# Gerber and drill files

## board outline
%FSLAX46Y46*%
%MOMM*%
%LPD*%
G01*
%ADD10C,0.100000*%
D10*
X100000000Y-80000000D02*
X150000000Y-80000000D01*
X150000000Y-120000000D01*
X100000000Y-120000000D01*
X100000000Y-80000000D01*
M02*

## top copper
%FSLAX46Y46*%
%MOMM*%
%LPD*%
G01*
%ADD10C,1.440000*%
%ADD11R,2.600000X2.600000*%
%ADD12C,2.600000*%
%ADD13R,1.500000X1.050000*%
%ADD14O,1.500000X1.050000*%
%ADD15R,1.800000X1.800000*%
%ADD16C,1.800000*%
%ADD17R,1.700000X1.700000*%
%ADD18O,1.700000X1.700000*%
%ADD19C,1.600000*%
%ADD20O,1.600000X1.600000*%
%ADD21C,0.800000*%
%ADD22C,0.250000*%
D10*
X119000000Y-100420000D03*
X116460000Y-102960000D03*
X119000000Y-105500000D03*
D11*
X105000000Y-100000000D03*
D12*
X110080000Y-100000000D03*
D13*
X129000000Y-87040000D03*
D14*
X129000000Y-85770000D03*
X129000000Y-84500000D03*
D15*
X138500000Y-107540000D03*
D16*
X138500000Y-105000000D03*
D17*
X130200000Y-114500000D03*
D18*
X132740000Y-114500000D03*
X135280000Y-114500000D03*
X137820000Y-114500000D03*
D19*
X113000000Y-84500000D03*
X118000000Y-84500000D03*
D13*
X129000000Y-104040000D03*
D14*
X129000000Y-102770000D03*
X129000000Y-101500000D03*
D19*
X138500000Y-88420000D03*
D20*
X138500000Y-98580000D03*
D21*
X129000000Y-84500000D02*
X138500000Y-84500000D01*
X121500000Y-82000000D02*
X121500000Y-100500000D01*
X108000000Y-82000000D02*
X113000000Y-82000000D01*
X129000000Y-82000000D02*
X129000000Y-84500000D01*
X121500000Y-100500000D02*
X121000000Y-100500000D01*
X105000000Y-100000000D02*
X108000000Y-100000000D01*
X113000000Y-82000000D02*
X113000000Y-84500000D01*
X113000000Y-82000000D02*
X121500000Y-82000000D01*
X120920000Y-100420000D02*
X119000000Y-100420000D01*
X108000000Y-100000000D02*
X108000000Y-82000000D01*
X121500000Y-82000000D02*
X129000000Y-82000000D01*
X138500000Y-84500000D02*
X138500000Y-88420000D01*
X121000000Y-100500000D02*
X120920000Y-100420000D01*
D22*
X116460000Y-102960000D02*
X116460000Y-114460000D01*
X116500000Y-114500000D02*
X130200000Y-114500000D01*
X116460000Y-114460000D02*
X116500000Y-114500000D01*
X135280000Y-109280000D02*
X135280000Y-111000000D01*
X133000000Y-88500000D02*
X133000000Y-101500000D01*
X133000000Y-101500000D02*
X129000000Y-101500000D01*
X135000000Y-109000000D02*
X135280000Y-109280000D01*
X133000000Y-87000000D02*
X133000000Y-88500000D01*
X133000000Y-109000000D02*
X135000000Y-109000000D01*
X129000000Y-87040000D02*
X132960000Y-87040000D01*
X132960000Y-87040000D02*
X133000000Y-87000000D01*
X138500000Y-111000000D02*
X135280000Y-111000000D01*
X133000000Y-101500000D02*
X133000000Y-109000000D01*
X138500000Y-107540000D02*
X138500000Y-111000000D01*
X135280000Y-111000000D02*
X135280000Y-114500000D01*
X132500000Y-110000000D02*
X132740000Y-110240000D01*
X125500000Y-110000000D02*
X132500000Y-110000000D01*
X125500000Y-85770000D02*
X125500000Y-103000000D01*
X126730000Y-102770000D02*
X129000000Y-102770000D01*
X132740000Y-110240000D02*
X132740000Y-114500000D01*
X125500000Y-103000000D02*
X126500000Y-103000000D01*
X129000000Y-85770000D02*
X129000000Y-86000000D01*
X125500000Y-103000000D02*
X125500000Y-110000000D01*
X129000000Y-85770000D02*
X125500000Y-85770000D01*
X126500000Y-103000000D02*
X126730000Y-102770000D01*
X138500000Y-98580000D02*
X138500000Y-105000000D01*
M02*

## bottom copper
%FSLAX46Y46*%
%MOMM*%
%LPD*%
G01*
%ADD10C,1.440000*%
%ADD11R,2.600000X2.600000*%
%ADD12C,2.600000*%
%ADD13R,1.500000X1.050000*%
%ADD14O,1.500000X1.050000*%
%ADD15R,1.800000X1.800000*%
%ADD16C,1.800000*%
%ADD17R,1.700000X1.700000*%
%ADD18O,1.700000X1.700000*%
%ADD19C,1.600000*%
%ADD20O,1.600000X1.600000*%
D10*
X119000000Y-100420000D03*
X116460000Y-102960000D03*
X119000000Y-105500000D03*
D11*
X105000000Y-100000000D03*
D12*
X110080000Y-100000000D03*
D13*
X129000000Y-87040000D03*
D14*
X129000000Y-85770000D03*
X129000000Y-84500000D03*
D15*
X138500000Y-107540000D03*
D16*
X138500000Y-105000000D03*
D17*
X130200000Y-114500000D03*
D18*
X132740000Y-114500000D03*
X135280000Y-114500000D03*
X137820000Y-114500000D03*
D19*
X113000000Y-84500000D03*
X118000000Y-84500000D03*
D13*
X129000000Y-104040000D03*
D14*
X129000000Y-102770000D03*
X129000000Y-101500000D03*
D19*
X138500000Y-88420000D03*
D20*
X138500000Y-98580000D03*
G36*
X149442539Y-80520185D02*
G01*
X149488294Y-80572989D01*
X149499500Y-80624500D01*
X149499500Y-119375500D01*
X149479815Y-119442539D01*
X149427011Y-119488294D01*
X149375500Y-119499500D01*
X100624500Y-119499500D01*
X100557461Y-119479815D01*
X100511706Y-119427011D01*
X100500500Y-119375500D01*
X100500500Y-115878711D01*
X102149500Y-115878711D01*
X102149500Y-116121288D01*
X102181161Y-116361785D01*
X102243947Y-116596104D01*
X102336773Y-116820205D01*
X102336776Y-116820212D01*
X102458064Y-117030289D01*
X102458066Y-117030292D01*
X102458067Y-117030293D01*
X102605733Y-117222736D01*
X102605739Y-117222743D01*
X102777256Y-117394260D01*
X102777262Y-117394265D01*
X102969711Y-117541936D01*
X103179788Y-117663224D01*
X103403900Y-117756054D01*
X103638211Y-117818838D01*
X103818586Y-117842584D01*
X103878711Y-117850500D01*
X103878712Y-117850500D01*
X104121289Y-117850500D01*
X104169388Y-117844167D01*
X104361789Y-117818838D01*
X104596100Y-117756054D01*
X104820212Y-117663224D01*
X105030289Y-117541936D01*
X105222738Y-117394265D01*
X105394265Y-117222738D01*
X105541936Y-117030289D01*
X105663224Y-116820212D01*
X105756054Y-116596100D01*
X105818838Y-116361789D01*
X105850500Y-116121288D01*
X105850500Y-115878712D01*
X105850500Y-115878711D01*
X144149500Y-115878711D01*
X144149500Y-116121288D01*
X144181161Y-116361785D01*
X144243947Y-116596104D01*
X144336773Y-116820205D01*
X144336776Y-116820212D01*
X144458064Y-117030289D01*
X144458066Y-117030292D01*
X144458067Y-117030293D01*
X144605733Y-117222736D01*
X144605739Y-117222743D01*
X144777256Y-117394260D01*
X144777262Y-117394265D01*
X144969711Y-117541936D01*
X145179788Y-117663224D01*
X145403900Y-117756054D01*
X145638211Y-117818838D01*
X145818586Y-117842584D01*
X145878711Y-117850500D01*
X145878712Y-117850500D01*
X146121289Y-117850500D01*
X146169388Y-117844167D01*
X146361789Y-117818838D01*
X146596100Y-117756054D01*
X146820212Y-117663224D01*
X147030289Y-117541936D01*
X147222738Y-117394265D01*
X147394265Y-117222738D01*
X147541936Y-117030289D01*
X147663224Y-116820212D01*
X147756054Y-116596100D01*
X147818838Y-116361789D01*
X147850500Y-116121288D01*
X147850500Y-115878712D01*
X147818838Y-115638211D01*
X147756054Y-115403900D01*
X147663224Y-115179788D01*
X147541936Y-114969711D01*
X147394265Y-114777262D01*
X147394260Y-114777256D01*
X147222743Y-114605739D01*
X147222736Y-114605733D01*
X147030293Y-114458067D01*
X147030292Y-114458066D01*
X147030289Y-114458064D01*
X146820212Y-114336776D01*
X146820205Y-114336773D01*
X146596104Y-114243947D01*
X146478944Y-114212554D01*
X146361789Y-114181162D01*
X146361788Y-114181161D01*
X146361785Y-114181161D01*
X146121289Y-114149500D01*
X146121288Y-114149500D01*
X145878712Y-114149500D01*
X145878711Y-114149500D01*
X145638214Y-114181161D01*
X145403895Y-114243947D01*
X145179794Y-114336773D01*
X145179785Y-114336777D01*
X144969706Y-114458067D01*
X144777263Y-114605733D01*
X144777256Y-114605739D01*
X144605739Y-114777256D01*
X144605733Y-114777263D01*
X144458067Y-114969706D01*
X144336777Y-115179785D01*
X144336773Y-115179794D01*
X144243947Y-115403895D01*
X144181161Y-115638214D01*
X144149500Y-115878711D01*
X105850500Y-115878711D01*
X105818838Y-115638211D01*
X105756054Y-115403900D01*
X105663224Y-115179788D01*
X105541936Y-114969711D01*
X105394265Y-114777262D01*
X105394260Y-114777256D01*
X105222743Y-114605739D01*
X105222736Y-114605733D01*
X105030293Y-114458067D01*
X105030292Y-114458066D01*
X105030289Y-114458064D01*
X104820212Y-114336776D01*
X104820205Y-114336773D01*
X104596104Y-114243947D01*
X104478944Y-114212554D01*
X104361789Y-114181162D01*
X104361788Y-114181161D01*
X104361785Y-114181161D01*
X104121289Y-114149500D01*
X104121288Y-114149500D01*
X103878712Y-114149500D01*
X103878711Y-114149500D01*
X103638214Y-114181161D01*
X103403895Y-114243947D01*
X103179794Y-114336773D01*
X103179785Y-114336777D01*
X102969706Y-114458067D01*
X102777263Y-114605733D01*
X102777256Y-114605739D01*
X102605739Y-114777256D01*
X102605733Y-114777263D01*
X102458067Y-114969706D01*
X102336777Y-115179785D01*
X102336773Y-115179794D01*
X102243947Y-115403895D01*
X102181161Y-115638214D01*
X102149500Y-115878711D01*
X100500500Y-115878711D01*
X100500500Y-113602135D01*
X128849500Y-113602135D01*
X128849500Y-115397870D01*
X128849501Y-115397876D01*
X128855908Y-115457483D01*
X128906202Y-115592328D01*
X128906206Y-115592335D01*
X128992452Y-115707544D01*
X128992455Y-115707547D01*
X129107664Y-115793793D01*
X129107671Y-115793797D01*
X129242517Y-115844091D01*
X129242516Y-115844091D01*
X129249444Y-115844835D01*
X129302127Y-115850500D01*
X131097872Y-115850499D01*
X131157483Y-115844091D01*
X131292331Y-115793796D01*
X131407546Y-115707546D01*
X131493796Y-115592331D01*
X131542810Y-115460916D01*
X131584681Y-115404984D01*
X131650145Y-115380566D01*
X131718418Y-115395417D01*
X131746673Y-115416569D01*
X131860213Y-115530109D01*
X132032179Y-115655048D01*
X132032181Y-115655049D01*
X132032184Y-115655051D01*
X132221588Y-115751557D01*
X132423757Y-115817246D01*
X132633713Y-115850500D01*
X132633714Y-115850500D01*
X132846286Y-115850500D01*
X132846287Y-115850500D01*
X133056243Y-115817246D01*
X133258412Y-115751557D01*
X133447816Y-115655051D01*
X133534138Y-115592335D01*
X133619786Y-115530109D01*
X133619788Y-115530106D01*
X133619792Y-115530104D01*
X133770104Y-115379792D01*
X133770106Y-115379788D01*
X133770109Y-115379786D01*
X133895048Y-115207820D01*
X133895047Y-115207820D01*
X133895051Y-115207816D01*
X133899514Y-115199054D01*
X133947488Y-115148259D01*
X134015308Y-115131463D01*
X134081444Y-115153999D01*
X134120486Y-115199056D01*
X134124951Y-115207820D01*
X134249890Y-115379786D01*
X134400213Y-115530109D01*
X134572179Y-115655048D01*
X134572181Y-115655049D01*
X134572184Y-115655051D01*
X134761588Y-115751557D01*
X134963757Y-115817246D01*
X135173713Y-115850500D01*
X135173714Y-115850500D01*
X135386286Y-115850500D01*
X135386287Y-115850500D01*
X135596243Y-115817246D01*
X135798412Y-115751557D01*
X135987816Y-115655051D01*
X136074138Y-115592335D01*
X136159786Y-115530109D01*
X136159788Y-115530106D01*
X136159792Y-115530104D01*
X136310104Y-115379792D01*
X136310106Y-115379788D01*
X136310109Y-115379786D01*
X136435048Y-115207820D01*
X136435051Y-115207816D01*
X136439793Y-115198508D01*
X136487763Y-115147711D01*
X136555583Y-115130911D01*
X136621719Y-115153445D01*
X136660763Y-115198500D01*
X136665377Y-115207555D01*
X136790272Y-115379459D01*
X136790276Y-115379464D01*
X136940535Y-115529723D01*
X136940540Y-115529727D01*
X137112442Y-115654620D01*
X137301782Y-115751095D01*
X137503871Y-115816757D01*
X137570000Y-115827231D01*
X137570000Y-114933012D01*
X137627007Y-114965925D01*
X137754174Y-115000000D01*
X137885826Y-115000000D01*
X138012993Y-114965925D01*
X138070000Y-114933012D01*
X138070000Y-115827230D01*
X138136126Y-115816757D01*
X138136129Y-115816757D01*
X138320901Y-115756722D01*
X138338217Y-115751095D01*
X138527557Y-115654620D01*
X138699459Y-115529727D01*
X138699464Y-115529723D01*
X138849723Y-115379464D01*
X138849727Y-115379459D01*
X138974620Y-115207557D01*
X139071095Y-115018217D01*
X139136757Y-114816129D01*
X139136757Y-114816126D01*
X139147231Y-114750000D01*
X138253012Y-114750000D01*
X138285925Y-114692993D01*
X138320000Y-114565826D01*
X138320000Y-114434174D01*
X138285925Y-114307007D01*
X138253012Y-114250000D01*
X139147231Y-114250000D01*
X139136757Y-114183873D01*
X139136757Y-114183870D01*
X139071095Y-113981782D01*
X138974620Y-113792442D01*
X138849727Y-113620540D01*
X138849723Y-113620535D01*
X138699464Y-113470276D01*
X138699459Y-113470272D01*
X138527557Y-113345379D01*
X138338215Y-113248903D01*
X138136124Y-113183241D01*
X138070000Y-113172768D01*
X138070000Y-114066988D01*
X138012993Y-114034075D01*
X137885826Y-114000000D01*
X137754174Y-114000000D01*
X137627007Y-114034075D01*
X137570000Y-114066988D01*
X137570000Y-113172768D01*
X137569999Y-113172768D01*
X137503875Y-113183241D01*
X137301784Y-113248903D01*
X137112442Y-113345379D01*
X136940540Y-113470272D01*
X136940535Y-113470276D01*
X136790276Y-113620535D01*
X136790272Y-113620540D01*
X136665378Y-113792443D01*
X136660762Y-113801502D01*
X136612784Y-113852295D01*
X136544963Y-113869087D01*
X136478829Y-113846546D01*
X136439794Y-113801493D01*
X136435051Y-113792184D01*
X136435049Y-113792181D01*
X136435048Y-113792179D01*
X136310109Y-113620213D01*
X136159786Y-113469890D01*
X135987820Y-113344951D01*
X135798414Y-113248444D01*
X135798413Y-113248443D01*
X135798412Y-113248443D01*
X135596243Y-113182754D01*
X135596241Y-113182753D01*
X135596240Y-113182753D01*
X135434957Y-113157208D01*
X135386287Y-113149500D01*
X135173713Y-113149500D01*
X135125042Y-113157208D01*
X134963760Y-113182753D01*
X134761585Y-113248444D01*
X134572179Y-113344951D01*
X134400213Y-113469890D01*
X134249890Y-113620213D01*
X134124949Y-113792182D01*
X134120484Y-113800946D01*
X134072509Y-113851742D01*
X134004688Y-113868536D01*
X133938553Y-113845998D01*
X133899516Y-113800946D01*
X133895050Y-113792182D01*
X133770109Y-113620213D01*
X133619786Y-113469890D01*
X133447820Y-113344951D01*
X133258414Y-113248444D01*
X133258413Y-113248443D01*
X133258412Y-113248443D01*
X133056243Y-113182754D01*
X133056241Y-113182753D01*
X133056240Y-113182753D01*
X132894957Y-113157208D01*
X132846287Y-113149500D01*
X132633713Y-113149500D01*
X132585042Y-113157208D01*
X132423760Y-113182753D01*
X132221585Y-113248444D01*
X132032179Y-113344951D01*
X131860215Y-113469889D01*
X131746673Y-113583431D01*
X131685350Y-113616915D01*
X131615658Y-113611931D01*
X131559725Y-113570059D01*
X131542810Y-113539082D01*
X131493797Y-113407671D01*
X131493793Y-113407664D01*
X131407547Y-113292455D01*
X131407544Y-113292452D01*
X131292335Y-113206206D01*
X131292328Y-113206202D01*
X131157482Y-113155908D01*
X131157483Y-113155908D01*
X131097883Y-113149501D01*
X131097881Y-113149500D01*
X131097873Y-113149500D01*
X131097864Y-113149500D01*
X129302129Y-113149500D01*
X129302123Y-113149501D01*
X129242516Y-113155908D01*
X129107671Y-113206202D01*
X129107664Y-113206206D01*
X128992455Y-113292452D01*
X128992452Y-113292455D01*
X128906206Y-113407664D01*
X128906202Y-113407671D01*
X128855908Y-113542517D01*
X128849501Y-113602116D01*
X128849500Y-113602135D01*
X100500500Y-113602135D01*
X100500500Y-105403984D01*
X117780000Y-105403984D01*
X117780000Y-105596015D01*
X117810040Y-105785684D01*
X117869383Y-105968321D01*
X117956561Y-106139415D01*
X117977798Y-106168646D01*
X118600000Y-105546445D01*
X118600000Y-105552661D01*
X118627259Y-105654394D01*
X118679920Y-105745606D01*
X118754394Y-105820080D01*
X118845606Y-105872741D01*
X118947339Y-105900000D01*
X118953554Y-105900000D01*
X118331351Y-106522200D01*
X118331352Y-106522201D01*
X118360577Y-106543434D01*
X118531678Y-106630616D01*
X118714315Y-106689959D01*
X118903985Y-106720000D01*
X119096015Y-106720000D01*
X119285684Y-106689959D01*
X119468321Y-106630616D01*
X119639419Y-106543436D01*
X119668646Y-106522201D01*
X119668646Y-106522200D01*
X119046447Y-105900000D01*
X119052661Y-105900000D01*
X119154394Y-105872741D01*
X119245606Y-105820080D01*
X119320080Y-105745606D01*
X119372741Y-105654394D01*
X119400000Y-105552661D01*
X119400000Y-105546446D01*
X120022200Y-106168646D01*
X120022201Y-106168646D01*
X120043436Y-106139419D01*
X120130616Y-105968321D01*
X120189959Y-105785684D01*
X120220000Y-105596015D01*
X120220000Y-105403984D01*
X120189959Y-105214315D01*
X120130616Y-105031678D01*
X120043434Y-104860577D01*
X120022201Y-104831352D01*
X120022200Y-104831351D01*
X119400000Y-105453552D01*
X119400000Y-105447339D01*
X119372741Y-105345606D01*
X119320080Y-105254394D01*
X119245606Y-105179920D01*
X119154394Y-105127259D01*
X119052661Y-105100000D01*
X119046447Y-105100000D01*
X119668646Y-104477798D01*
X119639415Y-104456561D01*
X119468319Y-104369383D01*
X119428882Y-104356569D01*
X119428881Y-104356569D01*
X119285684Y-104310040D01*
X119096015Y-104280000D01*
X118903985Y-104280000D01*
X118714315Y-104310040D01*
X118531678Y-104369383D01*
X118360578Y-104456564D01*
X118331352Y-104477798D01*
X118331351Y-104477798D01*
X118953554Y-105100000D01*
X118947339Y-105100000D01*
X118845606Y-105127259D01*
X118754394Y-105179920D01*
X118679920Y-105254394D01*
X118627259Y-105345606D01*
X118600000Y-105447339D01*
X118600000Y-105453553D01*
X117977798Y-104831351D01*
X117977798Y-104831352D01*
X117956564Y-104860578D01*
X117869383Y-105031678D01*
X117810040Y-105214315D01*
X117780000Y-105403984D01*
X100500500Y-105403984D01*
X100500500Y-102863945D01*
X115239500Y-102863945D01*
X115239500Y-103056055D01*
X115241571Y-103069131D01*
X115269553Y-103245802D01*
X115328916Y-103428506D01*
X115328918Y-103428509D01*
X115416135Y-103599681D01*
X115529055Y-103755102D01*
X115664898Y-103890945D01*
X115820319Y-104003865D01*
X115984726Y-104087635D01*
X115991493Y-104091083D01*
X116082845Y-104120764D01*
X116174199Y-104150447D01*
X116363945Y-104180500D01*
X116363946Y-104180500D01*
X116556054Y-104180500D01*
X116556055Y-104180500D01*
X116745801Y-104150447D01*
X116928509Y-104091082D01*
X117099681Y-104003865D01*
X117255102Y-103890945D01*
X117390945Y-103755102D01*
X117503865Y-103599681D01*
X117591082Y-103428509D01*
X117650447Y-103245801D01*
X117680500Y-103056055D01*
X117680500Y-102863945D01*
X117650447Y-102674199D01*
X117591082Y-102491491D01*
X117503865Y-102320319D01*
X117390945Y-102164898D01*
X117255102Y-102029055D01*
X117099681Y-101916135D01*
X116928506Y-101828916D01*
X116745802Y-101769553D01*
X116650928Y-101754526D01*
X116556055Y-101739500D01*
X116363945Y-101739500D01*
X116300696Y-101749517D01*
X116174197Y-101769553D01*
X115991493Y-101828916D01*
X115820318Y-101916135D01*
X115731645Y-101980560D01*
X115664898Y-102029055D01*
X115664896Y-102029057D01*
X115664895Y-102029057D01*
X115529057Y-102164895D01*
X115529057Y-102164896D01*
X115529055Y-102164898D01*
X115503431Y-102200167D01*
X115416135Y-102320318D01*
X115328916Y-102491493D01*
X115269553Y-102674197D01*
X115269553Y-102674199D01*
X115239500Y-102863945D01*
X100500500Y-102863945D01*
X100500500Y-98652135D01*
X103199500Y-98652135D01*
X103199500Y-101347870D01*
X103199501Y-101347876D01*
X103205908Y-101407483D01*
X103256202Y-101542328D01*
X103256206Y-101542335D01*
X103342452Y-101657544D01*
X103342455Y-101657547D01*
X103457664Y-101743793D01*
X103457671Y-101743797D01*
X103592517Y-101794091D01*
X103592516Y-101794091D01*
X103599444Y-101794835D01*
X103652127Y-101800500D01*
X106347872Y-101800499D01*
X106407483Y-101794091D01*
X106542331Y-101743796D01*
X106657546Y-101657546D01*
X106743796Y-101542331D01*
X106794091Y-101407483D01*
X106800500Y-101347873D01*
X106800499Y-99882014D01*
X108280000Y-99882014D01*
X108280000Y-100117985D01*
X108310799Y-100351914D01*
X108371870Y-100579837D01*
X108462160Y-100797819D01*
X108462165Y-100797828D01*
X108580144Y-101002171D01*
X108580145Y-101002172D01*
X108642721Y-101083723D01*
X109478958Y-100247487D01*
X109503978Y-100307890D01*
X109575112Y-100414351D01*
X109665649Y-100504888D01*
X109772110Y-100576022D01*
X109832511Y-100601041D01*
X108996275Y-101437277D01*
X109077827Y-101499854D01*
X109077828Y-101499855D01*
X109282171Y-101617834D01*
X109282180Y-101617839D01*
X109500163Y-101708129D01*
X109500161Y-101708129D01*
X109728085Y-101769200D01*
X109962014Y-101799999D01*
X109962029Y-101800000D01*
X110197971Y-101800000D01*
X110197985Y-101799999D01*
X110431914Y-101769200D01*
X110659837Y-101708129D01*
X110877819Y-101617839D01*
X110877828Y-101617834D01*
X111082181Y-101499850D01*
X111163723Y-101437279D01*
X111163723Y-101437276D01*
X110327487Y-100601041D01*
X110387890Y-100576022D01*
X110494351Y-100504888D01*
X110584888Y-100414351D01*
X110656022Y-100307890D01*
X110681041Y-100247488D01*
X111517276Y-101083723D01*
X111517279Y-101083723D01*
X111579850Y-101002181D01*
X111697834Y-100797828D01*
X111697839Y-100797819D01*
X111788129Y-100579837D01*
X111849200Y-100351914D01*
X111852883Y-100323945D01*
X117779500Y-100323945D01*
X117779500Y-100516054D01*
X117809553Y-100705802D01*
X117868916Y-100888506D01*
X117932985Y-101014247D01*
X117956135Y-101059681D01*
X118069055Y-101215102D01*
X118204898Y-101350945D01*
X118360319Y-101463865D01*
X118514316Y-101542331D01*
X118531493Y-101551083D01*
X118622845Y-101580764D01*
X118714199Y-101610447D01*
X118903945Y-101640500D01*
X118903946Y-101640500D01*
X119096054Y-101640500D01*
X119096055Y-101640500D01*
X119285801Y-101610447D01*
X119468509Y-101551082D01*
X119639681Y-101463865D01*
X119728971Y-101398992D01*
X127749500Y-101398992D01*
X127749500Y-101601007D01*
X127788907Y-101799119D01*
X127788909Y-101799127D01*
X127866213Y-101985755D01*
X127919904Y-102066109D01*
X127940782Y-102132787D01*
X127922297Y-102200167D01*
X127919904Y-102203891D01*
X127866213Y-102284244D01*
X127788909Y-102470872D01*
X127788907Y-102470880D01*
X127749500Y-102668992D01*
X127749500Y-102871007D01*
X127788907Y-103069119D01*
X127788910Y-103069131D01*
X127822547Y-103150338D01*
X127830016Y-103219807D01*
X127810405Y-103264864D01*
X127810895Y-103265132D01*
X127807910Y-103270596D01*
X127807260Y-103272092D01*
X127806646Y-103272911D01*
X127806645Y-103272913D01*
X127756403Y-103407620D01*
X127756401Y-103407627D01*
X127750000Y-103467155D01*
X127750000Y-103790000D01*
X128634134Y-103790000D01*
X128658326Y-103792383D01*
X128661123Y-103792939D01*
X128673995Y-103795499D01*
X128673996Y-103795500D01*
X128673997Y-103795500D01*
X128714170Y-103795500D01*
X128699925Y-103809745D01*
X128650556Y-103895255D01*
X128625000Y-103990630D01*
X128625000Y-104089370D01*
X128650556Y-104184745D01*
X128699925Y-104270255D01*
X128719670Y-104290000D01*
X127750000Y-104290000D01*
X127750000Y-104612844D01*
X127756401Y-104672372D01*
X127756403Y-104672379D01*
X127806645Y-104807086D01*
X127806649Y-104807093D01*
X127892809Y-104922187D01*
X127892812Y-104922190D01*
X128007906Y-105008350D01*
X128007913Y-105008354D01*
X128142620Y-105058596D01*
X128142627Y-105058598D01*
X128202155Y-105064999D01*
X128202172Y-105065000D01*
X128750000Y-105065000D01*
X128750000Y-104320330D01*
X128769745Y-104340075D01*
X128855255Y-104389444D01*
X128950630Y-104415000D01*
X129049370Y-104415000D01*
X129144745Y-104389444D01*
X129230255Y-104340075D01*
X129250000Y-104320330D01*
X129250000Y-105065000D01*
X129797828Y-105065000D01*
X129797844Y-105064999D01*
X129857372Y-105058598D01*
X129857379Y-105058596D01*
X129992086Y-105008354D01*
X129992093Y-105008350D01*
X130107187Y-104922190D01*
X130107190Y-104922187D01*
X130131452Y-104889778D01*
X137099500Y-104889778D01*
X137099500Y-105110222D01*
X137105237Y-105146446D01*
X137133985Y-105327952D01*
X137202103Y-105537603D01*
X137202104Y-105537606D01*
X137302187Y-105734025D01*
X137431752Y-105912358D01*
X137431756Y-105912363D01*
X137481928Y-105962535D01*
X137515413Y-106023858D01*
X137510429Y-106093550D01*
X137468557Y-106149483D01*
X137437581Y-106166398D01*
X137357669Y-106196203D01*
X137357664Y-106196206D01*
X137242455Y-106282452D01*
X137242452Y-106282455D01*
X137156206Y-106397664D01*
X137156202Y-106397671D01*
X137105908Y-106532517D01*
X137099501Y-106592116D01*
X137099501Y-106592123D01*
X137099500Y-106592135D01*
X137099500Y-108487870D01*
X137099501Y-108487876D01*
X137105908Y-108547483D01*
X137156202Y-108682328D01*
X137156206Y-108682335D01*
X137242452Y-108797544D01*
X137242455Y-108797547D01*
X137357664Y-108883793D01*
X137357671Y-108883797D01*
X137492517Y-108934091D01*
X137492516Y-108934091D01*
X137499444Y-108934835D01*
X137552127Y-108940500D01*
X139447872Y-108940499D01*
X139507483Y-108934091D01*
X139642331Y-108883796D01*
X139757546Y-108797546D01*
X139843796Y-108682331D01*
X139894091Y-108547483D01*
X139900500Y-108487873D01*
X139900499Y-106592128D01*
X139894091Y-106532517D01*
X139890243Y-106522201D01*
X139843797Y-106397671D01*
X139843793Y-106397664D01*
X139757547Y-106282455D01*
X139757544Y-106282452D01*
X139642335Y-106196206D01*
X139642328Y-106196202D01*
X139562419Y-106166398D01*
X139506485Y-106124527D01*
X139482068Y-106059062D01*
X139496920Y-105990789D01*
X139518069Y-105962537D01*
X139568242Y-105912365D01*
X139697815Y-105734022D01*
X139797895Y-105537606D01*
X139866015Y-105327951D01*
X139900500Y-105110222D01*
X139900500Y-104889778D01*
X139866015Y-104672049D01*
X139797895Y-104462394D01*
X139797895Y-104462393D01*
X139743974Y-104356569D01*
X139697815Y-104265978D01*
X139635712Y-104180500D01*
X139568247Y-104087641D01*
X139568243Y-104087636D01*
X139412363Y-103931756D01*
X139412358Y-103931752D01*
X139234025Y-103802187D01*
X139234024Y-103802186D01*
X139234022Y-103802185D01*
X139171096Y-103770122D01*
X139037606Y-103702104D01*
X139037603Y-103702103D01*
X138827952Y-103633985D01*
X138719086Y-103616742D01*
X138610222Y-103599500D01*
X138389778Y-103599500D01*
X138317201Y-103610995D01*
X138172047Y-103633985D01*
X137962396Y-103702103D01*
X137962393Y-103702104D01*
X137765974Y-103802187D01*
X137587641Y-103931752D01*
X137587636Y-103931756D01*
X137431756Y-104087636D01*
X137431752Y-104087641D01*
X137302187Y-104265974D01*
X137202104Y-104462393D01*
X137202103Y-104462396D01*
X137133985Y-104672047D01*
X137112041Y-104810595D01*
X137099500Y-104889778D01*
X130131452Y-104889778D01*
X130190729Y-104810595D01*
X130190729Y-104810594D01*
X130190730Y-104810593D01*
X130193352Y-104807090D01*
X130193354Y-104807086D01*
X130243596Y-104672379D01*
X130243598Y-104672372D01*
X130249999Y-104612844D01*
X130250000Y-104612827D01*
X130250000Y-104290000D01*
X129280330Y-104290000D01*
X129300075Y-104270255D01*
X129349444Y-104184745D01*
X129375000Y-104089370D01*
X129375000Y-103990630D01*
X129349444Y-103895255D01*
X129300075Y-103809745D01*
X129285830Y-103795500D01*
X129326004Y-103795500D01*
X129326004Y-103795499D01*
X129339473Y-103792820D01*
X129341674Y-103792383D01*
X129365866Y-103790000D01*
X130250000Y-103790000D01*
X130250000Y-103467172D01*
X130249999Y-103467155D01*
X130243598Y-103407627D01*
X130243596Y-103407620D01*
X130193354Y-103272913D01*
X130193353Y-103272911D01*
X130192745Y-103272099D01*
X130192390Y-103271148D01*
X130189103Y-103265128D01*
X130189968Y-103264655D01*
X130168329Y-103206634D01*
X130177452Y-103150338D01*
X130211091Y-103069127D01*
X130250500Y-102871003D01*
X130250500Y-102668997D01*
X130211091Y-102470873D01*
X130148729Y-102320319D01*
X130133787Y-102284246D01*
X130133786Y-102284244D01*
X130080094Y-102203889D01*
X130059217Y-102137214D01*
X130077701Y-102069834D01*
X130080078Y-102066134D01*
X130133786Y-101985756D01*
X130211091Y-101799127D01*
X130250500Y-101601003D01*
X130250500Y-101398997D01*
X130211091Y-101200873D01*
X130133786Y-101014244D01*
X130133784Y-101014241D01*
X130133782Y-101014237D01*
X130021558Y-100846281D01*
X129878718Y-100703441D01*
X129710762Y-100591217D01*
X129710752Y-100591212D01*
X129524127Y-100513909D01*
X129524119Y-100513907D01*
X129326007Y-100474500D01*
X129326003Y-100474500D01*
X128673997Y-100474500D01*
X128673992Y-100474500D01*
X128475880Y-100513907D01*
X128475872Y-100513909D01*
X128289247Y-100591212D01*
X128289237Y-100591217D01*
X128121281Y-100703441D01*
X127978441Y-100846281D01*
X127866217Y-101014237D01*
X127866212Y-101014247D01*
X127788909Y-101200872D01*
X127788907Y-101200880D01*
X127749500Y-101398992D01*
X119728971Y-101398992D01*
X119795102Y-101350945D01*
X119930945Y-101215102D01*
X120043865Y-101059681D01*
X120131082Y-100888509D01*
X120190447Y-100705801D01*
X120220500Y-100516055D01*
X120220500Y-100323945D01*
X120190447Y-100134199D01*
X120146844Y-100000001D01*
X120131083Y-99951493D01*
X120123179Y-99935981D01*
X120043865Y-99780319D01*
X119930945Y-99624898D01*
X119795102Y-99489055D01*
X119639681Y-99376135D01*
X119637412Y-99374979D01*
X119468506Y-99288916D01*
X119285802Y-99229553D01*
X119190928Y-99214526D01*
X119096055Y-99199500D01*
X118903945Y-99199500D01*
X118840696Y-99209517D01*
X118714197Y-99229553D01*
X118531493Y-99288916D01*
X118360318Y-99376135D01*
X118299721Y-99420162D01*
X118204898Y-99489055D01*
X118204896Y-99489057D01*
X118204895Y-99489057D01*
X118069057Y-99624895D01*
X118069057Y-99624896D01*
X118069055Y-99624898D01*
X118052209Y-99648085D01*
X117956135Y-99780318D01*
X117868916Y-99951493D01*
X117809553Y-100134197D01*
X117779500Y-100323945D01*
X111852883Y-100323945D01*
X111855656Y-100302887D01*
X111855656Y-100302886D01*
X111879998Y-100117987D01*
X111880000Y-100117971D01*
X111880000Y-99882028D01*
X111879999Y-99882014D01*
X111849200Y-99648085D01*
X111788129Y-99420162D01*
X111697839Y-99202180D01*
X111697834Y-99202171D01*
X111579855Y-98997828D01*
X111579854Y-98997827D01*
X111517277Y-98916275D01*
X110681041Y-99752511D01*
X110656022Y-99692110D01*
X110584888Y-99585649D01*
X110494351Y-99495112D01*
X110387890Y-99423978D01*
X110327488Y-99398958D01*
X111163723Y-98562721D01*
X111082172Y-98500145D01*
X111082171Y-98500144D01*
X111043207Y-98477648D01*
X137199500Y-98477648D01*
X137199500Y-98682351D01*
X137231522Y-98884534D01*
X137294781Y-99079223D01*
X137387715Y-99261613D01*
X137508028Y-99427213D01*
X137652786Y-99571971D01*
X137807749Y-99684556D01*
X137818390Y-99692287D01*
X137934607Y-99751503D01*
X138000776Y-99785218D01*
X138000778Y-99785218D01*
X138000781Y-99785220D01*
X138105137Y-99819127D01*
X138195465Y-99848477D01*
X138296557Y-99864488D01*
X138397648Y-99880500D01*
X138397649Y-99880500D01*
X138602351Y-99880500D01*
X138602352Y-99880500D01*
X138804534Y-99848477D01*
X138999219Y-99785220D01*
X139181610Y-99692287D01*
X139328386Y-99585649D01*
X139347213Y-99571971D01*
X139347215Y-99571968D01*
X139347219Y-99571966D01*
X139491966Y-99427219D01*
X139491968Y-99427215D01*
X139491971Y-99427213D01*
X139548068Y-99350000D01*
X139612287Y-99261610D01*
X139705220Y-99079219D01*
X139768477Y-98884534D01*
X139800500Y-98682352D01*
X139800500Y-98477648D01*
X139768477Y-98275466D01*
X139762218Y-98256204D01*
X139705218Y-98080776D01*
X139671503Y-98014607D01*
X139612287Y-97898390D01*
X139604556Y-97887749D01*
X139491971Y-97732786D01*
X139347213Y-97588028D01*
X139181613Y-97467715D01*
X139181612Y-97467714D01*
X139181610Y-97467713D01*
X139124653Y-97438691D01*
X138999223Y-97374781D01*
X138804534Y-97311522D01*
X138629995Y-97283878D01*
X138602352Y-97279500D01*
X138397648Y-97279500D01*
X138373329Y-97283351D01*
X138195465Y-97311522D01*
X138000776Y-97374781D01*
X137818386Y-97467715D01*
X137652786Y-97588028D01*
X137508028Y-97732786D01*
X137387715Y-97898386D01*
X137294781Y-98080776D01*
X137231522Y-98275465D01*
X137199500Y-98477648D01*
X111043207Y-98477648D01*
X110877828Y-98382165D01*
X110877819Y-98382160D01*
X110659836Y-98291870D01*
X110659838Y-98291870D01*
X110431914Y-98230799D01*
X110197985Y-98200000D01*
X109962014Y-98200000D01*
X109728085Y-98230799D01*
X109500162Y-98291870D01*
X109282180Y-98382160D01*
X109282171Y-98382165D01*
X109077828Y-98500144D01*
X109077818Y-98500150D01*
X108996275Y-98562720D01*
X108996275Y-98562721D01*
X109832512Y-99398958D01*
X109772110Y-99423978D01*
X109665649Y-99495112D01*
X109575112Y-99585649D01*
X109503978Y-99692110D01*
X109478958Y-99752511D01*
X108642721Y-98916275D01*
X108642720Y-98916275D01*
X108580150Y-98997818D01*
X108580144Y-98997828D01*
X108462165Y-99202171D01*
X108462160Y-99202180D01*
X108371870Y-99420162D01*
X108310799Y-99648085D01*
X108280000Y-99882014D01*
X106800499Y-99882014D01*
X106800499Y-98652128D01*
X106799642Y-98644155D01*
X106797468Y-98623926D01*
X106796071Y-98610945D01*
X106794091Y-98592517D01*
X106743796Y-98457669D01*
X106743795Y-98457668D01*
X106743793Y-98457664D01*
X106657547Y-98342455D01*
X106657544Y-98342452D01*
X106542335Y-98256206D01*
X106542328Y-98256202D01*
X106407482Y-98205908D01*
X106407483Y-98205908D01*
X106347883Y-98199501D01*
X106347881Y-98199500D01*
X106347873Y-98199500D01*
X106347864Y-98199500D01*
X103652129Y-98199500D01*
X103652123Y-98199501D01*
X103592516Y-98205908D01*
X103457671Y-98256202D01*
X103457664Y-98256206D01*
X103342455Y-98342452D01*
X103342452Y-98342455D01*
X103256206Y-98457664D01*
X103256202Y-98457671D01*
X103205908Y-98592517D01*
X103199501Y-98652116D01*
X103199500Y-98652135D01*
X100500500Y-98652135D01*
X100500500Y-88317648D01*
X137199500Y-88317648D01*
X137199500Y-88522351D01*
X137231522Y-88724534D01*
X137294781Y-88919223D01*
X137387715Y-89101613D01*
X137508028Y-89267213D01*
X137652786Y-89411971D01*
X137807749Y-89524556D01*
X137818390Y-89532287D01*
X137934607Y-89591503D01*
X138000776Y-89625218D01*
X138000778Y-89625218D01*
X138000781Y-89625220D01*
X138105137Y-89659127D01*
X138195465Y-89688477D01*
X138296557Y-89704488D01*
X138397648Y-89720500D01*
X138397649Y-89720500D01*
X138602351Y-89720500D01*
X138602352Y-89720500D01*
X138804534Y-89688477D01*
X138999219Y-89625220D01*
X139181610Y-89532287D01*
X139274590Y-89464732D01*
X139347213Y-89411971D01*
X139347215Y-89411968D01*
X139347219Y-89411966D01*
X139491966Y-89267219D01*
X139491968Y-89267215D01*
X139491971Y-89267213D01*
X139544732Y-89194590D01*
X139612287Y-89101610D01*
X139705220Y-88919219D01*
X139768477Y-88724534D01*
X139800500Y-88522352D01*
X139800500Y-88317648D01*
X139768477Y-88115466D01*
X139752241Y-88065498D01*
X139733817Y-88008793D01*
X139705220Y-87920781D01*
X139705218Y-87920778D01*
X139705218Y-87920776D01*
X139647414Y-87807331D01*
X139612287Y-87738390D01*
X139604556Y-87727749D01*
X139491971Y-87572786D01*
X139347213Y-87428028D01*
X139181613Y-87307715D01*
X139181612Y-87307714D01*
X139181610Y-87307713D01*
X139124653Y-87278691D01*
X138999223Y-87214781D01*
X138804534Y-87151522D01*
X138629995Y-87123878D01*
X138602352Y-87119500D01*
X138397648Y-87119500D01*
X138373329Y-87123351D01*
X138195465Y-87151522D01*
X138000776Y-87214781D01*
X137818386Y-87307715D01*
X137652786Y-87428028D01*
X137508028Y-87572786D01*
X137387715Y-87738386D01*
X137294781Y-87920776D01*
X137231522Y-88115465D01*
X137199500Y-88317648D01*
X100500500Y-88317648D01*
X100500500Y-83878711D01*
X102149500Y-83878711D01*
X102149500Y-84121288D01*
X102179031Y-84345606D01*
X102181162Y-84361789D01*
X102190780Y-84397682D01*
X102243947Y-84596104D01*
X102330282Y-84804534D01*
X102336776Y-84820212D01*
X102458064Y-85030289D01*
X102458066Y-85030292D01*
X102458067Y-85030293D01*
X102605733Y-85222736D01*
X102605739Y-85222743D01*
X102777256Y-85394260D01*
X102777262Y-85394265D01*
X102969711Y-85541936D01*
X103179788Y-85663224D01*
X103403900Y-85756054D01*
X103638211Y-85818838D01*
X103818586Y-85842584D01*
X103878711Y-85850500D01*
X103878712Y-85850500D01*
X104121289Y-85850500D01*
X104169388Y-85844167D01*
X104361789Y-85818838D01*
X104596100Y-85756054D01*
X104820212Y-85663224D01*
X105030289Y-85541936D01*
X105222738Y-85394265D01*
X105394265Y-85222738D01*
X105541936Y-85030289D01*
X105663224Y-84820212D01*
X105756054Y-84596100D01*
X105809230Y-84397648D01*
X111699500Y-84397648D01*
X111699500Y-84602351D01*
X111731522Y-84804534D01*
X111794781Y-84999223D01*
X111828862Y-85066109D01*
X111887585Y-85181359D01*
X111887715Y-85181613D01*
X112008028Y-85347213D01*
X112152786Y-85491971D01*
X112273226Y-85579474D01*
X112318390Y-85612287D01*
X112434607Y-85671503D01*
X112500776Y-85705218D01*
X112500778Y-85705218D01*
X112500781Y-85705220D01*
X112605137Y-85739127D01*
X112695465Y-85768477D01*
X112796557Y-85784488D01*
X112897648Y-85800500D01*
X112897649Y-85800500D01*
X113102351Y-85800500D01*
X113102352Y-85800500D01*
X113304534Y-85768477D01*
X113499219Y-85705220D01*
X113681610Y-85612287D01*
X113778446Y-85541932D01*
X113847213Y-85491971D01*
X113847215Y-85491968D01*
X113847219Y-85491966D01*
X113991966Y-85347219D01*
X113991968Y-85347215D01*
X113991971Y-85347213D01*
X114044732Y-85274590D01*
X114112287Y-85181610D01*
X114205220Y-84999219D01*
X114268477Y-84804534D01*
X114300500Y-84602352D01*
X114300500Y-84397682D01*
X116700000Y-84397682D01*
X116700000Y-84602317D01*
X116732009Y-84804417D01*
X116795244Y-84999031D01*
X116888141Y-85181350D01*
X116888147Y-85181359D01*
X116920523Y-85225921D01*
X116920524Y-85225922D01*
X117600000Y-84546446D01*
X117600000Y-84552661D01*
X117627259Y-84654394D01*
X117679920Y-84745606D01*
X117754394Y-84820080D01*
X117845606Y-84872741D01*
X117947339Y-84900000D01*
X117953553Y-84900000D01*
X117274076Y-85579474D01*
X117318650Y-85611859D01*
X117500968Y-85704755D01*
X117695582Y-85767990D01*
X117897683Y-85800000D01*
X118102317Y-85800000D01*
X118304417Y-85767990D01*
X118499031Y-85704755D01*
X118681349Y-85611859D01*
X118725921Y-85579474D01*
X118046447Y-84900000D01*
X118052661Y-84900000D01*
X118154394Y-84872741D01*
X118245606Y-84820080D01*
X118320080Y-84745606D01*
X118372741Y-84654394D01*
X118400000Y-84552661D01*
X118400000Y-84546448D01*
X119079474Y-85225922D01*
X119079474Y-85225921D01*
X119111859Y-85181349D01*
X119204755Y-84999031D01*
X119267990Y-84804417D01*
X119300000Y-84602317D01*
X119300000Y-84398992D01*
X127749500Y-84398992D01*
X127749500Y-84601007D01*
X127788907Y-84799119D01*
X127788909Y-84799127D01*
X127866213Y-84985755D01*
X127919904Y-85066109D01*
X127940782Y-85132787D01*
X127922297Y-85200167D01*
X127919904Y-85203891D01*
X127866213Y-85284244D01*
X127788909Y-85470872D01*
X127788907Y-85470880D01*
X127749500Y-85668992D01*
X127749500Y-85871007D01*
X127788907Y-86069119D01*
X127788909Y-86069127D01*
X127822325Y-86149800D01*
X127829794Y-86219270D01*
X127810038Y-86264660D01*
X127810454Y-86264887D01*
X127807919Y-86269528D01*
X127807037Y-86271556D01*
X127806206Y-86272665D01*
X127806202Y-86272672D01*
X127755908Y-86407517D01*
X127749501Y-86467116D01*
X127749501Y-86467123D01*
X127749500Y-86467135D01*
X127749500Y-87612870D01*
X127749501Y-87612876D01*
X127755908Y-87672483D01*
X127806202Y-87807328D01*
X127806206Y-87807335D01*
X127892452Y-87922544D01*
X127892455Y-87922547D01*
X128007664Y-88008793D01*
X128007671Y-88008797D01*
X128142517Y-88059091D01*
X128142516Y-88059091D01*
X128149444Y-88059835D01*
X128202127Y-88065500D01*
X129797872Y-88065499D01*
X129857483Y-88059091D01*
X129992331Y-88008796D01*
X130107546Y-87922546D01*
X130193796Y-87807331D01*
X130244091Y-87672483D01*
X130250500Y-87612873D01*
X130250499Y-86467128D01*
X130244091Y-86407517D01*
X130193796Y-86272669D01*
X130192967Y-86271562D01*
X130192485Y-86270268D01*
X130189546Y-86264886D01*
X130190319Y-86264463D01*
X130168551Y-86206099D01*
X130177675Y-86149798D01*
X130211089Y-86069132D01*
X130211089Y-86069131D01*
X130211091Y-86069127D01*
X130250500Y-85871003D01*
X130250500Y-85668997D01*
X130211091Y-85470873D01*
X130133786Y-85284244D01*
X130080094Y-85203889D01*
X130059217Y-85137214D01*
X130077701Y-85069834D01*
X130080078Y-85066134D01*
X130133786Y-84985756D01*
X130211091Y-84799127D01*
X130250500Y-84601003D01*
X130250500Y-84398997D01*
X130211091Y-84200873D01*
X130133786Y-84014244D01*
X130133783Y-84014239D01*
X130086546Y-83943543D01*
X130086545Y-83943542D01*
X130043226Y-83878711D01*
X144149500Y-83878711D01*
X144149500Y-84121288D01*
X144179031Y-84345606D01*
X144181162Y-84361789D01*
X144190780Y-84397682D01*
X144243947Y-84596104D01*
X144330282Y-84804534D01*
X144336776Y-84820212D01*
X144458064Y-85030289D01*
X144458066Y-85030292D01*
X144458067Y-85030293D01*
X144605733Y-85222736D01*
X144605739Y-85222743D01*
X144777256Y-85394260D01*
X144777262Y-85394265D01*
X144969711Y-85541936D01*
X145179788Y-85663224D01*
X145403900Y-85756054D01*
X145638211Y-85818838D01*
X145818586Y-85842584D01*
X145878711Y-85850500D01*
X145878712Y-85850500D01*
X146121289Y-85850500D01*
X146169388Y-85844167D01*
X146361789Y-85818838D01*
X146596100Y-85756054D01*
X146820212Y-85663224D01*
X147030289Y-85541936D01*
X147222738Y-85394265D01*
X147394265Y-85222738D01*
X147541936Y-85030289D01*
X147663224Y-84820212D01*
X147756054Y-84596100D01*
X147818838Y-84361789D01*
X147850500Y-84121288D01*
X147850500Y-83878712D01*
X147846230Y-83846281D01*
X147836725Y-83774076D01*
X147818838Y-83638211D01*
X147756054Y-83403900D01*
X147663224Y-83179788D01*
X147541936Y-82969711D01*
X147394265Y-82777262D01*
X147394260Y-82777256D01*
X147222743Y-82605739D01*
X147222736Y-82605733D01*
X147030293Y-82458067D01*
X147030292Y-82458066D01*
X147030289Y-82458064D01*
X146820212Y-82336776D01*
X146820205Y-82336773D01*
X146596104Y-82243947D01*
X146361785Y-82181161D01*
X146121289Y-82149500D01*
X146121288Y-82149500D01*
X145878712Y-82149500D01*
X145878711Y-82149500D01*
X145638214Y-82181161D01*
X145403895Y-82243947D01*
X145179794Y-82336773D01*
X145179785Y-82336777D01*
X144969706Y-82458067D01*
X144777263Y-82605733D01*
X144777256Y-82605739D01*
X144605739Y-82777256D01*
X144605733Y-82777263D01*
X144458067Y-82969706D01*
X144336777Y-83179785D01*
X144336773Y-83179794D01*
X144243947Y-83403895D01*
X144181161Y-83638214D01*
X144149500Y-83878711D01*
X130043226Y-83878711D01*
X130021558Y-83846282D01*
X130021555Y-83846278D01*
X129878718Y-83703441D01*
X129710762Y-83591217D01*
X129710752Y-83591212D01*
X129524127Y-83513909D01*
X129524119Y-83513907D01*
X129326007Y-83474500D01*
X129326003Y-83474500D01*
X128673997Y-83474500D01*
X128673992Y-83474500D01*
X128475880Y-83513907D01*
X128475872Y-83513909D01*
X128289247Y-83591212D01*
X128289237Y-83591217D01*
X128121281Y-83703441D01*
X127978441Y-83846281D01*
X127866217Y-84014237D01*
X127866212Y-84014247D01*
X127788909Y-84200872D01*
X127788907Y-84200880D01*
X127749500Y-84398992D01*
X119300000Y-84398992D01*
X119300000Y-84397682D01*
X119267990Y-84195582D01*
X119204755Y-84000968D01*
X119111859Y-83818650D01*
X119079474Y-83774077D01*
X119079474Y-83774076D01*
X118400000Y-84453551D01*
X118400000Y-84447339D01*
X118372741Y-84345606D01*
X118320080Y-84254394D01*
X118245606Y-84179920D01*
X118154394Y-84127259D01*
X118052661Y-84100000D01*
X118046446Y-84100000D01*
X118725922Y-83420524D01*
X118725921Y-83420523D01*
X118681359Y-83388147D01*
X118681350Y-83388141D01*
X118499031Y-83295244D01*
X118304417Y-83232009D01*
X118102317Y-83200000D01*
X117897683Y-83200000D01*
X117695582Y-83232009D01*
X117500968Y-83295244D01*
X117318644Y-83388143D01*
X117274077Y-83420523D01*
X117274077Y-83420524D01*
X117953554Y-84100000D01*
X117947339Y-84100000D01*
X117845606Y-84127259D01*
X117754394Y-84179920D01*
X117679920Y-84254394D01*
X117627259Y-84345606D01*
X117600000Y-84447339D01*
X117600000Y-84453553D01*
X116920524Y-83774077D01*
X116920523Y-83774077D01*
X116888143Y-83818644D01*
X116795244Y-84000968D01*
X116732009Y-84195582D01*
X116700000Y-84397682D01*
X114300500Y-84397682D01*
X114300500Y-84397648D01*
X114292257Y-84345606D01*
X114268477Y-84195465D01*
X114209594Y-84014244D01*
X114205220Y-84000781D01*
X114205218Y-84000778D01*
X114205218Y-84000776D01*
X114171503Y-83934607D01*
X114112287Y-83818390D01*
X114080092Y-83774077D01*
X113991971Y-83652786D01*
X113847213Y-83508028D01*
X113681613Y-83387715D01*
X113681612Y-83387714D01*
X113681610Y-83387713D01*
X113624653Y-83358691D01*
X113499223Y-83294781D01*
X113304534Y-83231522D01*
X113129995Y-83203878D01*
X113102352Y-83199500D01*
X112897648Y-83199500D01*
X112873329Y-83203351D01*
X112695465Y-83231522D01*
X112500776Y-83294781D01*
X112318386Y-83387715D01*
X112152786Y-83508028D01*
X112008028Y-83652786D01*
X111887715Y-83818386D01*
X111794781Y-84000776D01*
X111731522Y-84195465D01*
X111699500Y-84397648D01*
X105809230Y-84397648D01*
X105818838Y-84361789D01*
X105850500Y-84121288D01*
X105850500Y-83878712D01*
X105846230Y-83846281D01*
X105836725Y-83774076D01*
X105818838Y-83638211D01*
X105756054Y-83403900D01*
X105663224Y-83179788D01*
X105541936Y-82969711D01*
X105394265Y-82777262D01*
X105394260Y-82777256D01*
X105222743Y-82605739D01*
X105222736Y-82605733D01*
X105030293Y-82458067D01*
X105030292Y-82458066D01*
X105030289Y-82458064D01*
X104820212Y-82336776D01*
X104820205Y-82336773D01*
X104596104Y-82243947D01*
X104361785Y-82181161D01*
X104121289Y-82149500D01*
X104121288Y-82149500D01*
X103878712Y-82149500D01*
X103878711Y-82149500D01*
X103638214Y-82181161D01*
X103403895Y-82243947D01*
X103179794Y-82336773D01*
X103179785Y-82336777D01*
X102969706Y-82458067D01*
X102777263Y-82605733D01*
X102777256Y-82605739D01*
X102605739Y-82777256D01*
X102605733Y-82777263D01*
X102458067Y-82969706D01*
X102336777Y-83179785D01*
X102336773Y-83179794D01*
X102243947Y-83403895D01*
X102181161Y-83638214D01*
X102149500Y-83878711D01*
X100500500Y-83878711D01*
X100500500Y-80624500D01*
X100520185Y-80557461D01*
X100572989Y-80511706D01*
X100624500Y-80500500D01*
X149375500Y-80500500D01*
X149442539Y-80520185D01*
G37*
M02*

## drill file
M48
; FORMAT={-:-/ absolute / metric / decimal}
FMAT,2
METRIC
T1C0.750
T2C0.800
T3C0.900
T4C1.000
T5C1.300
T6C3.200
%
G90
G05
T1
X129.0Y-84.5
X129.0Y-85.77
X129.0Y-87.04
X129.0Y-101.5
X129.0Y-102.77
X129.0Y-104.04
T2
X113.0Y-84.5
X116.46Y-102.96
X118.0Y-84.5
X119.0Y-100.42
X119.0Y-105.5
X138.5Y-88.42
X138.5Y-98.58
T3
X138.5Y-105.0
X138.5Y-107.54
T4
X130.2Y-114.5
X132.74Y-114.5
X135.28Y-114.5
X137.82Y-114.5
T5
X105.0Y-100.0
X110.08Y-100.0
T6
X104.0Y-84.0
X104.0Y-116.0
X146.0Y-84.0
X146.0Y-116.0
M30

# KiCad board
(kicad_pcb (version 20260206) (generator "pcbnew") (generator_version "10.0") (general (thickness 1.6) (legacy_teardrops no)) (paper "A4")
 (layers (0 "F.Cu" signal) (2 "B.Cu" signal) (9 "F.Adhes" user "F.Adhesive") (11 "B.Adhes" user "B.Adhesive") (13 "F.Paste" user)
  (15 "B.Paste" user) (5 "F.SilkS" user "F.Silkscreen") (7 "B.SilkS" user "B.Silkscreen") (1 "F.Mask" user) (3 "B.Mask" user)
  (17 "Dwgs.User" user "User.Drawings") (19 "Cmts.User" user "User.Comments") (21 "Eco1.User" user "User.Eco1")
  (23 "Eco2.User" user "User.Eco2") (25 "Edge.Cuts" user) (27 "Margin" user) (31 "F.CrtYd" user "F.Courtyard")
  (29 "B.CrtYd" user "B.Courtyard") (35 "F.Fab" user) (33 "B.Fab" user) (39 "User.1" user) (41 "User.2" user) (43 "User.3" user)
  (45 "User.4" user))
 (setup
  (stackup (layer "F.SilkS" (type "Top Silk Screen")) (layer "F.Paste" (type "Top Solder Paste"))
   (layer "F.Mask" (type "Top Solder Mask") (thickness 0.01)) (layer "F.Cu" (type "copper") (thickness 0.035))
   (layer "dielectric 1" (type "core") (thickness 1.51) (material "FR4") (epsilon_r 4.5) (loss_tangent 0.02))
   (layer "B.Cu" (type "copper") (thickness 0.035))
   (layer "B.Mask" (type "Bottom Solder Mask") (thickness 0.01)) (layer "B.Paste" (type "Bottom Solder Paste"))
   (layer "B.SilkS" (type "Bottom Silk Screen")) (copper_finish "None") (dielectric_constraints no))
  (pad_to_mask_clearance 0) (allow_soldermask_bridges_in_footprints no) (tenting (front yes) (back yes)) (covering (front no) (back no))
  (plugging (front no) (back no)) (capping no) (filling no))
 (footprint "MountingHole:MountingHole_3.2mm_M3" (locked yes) (layer "F.Cu") (at 146 84)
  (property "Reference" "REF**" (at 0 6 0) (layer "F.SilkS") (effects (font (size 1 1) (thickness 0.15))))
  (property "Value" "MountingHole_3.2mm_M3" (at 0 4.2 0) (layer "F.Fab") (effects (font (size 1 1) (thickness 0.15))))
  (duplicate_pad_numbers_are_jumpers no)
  (pad "" np_thru_hole circle (at 0 0) (size 3.2 3.2) (drill 3.2) (layers "*.Cu" "*.Mask")))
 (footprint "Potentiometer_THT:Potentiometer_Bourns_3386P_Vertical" (layer "F.Cu") (at 119 100.42 180)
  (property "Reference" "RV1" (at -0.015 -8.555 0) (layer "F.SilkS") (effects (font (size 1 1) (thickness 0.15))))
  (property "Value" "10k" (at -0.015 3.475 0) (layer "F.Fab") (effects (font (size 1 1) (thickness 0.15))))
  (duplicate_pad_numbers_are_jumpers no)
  (pad "1" thru_hole circle (at 0 0 180) (size 1.44 1.44) (drill 0.8) (layers "*.Cu" "*.Mask") (remove_unused_layers no) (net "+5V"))
  (pad "2" thru_hole circle (at 2.54 -2.54 180) (size 1.44 1.44) (drill 0.8) (layers "*.Cu" "*.Mask") (remove_unused_layers no)
   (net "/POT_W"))
  (pad "3" thru_hole circle (at 0 -5.08 180) (size 1.44 1.44) (drill 0.8) (layers "*.Cu" "*.Mask") (remove_unused_layers no) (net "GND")))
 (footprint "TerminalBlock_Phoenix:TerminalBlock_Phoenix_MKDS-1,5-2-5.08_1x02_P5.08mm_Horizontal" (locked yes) (layer "F.Cu") (at 105 100)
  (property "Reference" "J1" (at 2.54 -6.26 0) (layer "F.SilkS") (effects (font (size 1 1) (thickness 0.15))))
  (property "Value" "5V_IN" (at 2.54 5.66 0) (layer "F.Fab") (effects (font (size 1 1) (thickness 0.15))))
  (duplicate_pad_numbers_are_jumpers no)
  (pad "1" thru_hole rect (at 0 0) (size 2.6 2.6) (drill 1.3) (layers "*.Cu" "*.Mask") (remove_unused_layers no) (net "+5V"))
  (pad "2" thru_hole circle (at 5.08 0) (size 2.6 2.6) (drill 1.3) (layers "*.Cu" "*.Mask") (remove_unused_layers no) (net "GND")))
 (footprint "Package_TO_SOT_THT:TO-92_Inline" (layer "F.Cu") (at 129 87.04 90)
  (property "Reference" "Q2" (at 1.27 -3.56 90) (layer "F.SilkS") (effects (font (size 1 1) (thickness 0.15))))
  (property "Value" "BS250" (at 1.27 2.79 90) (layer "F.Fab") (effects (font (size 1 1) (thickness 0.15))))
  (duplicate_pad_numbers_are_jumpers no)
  (pad "1" thru_hole rect (at 0 0 90) (size 1.05 1.5) (drill 0.75) (layers "*.Cu" "*.Mask") (remove_unused_layers no) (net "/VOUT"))
  (pad "2" thru_hole oval (at 1.27 0 90) (size 1.05 1.5) (drill 0.75) (layers "*.Cu" "*.Mask") (remove_unused_layers no) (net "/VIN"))
  (pad "3" thru_hole oval (at 2.54 0 90) (size 1.05 1.5) (drill 0.75) (layers "*.Cu" "*.Mask") (remove_unused_layers no) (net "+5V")))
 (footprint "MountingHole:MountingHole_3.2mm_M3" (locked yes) (layer "F.Cu") (at 104 84)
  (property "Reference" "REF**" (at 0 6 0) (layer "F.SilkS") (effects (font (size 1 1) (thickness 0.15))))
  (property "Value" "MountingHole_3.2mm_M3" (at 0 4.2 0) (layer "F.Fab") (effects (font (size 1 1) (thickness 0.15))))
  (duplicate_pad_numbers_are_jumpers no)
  (pad "" np_thru_hole circle (at 0 0) (size 3.2 3.2) (drill 3.2) (layers "*.Cu" "*.Mask")))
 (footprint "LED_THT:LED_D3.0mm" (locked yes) (layer "F.Cu") (at 138.5 107.54 90)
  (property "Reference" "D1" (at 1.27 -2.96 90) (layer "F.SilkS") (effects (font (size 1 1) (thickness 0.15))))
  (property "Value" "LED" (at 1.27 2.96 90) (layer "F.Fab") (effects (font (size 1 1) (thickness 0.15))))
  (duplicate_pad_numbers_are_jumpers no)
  (pad "1" thru_hole rect (at 0 0 90) (size 1.8 1.8) (drill 0.9) (layers "*.Cu" "*.Mask") (remove_unused_layers no) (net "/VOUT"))
  (pad "2" thru_hole circle (at 2.54 0 90) (size 1.8 1.8) (drill 0.9) (layers "*.Cu" "*.Mask") (remove_unused_layers no) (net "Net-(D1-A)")))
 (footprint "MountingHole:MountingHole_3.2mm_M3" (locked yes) (layer "F.Cu") (at 104 116)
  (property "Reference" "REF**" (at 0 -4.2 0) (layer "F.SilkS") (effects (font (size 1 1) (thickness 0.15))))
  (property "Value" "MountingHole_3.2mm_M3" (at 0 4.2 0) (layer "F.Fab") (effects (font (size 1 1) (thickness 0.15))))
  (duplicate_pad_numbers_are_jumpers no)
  (pad "" np_thru_hole circle (at 0 0) (size 3.2 3.2) (drill 3.2) (layers "*.Cu" "*.Mask")))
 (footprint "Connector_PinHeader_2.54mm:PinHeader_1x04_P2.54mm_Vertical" (layer "F.Cu") (at 130.2 114.5 90)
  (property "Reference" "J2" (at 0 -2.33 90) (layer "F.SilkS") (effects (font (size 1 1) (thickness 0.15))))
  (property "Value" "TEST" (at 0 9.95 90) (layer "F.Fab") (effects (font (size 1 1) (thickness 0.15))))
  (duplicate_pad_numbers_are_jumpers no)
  (pad "1" thru_hole rect (at 0 0 90) (size 1.7 1.7) (drill 1) (layers "*.Cu" "*.Mask") (remove_unused_layers no) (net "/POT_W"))
  (pad "2" thru_hole oval (at 0 2.54 90) (size 1.7 1.7) (drill 1) (layers "*.Cu" "*.Mask") (remove_unused_layers no) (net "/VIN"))
  (pad "3" thru_hole oval (at 0 5.08 90) (size 1.7 1.7) (drill 1) (layers "*.Cu" "*.Mask") (remove_unused_layers no) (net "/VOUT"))
  (pad "4" thru_hole oval (at 0 7.62 90) (size 1.7 1.7) (drill 1) (layers "*.Cu" "*.Mask") (remove_unused_layers no) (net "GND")))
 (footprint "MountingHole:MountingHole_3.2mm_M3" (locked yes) (layer "F.Cu") (at 146 116)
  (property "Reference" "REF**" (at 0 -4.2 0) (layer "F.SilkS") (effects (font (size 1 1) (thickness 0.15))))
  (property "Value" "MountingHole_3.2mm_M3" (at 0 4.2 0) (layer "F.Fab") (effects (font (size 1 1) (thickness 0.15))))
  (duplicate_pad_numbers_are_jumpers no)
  (pad "" np_thru_hole circle (at 0 0) (size 3.2 3.2) (drill 3.2) (layers "*.Cu" "*.Mask")))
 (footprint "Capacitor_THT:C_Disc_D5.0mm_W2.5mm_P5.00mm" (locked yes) (layer "F.Cu") (at 113 84.5)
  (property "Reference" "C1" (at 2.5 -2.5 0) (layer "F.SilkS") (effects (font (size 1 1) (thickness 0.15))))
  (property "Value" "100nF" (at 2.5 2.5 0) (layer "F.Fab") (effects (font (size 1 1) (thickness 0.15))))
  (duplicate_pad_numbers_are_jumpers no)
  (pad "1" thru_hole circle (at 0 0) (size 1.6 1.6) (drill 0.8) (layers "*.Cu" "*.Mask") (remove_unused_layers no) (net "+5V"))
  (pad "2" thru_hole circle (at 5 0) (size 1.6 1.6) (drill 0.8) (layers "*.Cu" "*.Mask") (remove_unused_layers no) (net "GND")))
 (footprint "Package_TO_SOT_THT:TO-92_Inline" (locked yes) (layer "F.Cu") (at 129 104.04 90)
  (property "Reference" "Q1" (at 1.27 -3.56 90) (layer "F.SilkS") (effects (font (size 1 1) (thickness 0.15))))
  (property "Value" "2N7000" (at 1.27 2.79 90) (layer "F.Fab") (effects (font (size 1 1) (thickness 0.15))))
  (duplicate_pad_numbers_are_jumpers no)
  (pad "1" thru_hole rect (at 0 0 90) (size 1.05 1.5) (drill 0.75) (layers "*.Cu" "*.Mask") (remove_unused_layers no) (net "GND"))
  (pad "2" thru_hole oval (at 1.27 0 90) (size 1.05 1.5) (drill 0.75) (layers "*.Cu" "*.Mask") (remove_unused_layers no) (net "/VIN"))
  (pad "3" thru_hole oval (at 2.54 0 90) (size 1.05 1.5) (drill 0.75) (layers "*.Cu" "*.Mask") (remove_unused_layers no) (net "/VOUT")))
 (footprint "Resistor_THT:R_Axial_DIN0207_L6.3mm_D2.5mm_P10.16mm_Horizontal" (layer "F.Cu") (at 138.5 88.42 -90)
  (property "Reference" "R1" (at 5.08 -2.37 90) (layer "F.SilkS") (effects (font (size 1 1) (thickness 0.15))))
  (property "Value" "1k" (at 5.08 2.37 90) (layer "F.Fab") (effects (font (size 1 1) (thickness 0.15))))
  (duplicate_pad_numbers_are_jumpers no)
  (pad "1" thru_hole circle (at 0 0 270) (size 1.6 1.6) (drill 0.8) (layers "*.Cu" "*.Mask") (remove_unused_layers no) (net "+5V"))
  (pad "2" thru_hole oval (at 10.16 0 270) (size 1.6 1.6) (drill 0.8) (layers "*.Cu" "*.Mask") (remove_unused_layers no) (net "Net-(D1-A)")))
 (gr_rect (start 100 80) (end 150 120) (stroke (width 0.1) (type solid)) (fill no) (layer "Edge.Cuts"))
 (segment (start 129 84.5) (end 138.5 84.5) (width 0.8) (layer "F.Cu") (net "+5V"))
 (segment (start 121.5 82) (end 121.5 100.5) (width 0.8) (layer "F.Cu") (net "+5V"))
 (segment (start 108 82) (end 113 82) (width 0.8) (layer "F.Cu") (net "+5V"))
 (segment (start 129 82) (end 129 84.5) (width 0.8) (layer "F.Cu") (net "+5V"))
 (segment (start 121.5 100.5) (end 121 100.5) (width 0.8) (layer "F.Cu") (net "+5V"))
 (segment (start 105 100) (end 108 100) (width 0.8) (layer "F.Cu") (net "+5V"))
 (segment (start 113 82) (end 113 84.5) (width 0.8) (layer "F.Cu") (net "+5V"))
 (segment (start 113 82) (end 121.5 82) (width 0.8) (layer "F.Cu") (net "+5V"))
 (segment (start 120.92 100.42) (end 119 100.42) (width 0.8) (layer "F.Cu") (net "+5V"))
 (segment (start 108 100) (end 108 82) (width 0.8) (layer "F.Cu") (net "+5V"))
 (segment (start 121.5 82) (end 129 82) (width 0.8) (layer "F.Cu") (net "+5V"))
 (segment (start 138.5 84.5) (end 138.5 88.42) (width 0.8) (layer "F.Cu") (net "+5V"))
 (segment (start 121 100.5) (end 120.92 100.42) (width 0.8) (layer "F.Cu") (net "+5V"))
 (segment (start 116.46 102.96) (end 116.46 114.46) (width 0.25) (layer "F.Cu") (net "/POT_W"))
 (segment (start 116.5 114.5) (end 130.2 114.5) (width 0.25) (layer "F.Cu") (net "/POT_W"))
 (segment (start 116.46 114.46) (end 116.5 114.5) (width 0.25) (layer "F.Cu") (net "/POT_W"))
 (segment (start 135.28 109.28) (end 135.28 111) (width 0.25) (layer "F.Cu") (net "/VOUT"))
 (segment (start 133 88.5) (end 133 101.5) (width 0.25) (layer "F.Cu") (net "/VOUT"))
 (segment (start 133 101.5) (end 129 101.5) (width 0.25) (layer "F.Cu") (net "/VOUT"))
 (segment (start 135 109) (end 135.28 109.28) (width 0.25) (layer "F.Cu") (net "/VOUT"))
 (segment (start 133 87) (end 133 88.5) (width 0.25) (layer "F.Cu") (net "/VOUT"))
 (segment (start 133 109) (end 135 109) (width 0.25) (layer "F.Cu") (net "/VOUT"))
 (segment (start 129 87.04) (end 132.96 87.04) (width 0.25) (layer "F.Cu") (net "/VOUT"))
 (segment (start 132.96 87.04) (end 133 87) (width 0.25) (layer "F.Cu") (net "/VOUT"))
 (segment (start 138.5 111) (end 135.28 111) (width 0.25) (layer "F.Cu") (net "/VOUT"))
 (segment (start 133 101.5) (end 133 109) (width 0.25) (layer "F.Cu") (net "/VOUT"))
 (segment (start 138.5 107.54) (end 138.5 111) (width 0.25) (layer "F.Cu") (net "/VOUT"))
 (segment (start 135.28 111) (end 135.28 114.5) (width 0.25) (layer "F.Cu") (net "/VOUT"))
 (segment (start 132.5 110) (end 132.74 110.24) (width 0.25) (layer "F.Cu") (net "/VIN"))
 (segment (start 125.5 110) (end 132.5 110) (width 0.25) (layer "F.Cu") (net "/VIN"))
 (segment (start 125.5 85.77) (end 125.5 103) (width 0.25) (layer "F.Cu") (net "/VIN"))
 (segment (start 126.73 102.77) (end 129 102.77) (width 0.25) (layer "F.Cu") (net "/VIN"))
 (segment (start 132.74 110.24) (end 132.74 114.5) (width 0.25) (layer "F.Cu") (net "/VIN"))
 (segment (start 125.5 103) (end 126.5 103) (width 0.25) (layer "F.Cu") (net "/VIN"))
 (segment (start 129 85.77) (end 129 86) (width 0.25) (layer "F.Cu") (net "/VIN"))
 (segment (start 125.5 103) (end 125.5 110) (width 0.25) (layer "F.Cu") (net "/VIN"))
 (segment (start 129 85.77) (end 125.5 85.77) (width 0.25) (layer "F.Cu") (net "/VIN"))
 (segment (start 126.5 103) (end 126.73 102.77) (width 0.25) (layer "F.Cu") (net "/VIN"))
 (segment (start 138.5 98.58) (end 138.5 105) (width 0.25) (layer "F.Cu") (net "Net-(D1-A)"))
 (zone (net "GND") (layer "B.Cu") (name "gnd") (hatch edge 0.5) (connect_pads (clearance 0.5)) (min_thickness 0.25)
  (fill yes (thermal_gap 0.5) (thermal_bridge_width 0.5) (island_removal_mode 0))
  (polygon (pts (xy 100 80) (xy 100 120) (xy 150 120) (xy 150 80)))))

